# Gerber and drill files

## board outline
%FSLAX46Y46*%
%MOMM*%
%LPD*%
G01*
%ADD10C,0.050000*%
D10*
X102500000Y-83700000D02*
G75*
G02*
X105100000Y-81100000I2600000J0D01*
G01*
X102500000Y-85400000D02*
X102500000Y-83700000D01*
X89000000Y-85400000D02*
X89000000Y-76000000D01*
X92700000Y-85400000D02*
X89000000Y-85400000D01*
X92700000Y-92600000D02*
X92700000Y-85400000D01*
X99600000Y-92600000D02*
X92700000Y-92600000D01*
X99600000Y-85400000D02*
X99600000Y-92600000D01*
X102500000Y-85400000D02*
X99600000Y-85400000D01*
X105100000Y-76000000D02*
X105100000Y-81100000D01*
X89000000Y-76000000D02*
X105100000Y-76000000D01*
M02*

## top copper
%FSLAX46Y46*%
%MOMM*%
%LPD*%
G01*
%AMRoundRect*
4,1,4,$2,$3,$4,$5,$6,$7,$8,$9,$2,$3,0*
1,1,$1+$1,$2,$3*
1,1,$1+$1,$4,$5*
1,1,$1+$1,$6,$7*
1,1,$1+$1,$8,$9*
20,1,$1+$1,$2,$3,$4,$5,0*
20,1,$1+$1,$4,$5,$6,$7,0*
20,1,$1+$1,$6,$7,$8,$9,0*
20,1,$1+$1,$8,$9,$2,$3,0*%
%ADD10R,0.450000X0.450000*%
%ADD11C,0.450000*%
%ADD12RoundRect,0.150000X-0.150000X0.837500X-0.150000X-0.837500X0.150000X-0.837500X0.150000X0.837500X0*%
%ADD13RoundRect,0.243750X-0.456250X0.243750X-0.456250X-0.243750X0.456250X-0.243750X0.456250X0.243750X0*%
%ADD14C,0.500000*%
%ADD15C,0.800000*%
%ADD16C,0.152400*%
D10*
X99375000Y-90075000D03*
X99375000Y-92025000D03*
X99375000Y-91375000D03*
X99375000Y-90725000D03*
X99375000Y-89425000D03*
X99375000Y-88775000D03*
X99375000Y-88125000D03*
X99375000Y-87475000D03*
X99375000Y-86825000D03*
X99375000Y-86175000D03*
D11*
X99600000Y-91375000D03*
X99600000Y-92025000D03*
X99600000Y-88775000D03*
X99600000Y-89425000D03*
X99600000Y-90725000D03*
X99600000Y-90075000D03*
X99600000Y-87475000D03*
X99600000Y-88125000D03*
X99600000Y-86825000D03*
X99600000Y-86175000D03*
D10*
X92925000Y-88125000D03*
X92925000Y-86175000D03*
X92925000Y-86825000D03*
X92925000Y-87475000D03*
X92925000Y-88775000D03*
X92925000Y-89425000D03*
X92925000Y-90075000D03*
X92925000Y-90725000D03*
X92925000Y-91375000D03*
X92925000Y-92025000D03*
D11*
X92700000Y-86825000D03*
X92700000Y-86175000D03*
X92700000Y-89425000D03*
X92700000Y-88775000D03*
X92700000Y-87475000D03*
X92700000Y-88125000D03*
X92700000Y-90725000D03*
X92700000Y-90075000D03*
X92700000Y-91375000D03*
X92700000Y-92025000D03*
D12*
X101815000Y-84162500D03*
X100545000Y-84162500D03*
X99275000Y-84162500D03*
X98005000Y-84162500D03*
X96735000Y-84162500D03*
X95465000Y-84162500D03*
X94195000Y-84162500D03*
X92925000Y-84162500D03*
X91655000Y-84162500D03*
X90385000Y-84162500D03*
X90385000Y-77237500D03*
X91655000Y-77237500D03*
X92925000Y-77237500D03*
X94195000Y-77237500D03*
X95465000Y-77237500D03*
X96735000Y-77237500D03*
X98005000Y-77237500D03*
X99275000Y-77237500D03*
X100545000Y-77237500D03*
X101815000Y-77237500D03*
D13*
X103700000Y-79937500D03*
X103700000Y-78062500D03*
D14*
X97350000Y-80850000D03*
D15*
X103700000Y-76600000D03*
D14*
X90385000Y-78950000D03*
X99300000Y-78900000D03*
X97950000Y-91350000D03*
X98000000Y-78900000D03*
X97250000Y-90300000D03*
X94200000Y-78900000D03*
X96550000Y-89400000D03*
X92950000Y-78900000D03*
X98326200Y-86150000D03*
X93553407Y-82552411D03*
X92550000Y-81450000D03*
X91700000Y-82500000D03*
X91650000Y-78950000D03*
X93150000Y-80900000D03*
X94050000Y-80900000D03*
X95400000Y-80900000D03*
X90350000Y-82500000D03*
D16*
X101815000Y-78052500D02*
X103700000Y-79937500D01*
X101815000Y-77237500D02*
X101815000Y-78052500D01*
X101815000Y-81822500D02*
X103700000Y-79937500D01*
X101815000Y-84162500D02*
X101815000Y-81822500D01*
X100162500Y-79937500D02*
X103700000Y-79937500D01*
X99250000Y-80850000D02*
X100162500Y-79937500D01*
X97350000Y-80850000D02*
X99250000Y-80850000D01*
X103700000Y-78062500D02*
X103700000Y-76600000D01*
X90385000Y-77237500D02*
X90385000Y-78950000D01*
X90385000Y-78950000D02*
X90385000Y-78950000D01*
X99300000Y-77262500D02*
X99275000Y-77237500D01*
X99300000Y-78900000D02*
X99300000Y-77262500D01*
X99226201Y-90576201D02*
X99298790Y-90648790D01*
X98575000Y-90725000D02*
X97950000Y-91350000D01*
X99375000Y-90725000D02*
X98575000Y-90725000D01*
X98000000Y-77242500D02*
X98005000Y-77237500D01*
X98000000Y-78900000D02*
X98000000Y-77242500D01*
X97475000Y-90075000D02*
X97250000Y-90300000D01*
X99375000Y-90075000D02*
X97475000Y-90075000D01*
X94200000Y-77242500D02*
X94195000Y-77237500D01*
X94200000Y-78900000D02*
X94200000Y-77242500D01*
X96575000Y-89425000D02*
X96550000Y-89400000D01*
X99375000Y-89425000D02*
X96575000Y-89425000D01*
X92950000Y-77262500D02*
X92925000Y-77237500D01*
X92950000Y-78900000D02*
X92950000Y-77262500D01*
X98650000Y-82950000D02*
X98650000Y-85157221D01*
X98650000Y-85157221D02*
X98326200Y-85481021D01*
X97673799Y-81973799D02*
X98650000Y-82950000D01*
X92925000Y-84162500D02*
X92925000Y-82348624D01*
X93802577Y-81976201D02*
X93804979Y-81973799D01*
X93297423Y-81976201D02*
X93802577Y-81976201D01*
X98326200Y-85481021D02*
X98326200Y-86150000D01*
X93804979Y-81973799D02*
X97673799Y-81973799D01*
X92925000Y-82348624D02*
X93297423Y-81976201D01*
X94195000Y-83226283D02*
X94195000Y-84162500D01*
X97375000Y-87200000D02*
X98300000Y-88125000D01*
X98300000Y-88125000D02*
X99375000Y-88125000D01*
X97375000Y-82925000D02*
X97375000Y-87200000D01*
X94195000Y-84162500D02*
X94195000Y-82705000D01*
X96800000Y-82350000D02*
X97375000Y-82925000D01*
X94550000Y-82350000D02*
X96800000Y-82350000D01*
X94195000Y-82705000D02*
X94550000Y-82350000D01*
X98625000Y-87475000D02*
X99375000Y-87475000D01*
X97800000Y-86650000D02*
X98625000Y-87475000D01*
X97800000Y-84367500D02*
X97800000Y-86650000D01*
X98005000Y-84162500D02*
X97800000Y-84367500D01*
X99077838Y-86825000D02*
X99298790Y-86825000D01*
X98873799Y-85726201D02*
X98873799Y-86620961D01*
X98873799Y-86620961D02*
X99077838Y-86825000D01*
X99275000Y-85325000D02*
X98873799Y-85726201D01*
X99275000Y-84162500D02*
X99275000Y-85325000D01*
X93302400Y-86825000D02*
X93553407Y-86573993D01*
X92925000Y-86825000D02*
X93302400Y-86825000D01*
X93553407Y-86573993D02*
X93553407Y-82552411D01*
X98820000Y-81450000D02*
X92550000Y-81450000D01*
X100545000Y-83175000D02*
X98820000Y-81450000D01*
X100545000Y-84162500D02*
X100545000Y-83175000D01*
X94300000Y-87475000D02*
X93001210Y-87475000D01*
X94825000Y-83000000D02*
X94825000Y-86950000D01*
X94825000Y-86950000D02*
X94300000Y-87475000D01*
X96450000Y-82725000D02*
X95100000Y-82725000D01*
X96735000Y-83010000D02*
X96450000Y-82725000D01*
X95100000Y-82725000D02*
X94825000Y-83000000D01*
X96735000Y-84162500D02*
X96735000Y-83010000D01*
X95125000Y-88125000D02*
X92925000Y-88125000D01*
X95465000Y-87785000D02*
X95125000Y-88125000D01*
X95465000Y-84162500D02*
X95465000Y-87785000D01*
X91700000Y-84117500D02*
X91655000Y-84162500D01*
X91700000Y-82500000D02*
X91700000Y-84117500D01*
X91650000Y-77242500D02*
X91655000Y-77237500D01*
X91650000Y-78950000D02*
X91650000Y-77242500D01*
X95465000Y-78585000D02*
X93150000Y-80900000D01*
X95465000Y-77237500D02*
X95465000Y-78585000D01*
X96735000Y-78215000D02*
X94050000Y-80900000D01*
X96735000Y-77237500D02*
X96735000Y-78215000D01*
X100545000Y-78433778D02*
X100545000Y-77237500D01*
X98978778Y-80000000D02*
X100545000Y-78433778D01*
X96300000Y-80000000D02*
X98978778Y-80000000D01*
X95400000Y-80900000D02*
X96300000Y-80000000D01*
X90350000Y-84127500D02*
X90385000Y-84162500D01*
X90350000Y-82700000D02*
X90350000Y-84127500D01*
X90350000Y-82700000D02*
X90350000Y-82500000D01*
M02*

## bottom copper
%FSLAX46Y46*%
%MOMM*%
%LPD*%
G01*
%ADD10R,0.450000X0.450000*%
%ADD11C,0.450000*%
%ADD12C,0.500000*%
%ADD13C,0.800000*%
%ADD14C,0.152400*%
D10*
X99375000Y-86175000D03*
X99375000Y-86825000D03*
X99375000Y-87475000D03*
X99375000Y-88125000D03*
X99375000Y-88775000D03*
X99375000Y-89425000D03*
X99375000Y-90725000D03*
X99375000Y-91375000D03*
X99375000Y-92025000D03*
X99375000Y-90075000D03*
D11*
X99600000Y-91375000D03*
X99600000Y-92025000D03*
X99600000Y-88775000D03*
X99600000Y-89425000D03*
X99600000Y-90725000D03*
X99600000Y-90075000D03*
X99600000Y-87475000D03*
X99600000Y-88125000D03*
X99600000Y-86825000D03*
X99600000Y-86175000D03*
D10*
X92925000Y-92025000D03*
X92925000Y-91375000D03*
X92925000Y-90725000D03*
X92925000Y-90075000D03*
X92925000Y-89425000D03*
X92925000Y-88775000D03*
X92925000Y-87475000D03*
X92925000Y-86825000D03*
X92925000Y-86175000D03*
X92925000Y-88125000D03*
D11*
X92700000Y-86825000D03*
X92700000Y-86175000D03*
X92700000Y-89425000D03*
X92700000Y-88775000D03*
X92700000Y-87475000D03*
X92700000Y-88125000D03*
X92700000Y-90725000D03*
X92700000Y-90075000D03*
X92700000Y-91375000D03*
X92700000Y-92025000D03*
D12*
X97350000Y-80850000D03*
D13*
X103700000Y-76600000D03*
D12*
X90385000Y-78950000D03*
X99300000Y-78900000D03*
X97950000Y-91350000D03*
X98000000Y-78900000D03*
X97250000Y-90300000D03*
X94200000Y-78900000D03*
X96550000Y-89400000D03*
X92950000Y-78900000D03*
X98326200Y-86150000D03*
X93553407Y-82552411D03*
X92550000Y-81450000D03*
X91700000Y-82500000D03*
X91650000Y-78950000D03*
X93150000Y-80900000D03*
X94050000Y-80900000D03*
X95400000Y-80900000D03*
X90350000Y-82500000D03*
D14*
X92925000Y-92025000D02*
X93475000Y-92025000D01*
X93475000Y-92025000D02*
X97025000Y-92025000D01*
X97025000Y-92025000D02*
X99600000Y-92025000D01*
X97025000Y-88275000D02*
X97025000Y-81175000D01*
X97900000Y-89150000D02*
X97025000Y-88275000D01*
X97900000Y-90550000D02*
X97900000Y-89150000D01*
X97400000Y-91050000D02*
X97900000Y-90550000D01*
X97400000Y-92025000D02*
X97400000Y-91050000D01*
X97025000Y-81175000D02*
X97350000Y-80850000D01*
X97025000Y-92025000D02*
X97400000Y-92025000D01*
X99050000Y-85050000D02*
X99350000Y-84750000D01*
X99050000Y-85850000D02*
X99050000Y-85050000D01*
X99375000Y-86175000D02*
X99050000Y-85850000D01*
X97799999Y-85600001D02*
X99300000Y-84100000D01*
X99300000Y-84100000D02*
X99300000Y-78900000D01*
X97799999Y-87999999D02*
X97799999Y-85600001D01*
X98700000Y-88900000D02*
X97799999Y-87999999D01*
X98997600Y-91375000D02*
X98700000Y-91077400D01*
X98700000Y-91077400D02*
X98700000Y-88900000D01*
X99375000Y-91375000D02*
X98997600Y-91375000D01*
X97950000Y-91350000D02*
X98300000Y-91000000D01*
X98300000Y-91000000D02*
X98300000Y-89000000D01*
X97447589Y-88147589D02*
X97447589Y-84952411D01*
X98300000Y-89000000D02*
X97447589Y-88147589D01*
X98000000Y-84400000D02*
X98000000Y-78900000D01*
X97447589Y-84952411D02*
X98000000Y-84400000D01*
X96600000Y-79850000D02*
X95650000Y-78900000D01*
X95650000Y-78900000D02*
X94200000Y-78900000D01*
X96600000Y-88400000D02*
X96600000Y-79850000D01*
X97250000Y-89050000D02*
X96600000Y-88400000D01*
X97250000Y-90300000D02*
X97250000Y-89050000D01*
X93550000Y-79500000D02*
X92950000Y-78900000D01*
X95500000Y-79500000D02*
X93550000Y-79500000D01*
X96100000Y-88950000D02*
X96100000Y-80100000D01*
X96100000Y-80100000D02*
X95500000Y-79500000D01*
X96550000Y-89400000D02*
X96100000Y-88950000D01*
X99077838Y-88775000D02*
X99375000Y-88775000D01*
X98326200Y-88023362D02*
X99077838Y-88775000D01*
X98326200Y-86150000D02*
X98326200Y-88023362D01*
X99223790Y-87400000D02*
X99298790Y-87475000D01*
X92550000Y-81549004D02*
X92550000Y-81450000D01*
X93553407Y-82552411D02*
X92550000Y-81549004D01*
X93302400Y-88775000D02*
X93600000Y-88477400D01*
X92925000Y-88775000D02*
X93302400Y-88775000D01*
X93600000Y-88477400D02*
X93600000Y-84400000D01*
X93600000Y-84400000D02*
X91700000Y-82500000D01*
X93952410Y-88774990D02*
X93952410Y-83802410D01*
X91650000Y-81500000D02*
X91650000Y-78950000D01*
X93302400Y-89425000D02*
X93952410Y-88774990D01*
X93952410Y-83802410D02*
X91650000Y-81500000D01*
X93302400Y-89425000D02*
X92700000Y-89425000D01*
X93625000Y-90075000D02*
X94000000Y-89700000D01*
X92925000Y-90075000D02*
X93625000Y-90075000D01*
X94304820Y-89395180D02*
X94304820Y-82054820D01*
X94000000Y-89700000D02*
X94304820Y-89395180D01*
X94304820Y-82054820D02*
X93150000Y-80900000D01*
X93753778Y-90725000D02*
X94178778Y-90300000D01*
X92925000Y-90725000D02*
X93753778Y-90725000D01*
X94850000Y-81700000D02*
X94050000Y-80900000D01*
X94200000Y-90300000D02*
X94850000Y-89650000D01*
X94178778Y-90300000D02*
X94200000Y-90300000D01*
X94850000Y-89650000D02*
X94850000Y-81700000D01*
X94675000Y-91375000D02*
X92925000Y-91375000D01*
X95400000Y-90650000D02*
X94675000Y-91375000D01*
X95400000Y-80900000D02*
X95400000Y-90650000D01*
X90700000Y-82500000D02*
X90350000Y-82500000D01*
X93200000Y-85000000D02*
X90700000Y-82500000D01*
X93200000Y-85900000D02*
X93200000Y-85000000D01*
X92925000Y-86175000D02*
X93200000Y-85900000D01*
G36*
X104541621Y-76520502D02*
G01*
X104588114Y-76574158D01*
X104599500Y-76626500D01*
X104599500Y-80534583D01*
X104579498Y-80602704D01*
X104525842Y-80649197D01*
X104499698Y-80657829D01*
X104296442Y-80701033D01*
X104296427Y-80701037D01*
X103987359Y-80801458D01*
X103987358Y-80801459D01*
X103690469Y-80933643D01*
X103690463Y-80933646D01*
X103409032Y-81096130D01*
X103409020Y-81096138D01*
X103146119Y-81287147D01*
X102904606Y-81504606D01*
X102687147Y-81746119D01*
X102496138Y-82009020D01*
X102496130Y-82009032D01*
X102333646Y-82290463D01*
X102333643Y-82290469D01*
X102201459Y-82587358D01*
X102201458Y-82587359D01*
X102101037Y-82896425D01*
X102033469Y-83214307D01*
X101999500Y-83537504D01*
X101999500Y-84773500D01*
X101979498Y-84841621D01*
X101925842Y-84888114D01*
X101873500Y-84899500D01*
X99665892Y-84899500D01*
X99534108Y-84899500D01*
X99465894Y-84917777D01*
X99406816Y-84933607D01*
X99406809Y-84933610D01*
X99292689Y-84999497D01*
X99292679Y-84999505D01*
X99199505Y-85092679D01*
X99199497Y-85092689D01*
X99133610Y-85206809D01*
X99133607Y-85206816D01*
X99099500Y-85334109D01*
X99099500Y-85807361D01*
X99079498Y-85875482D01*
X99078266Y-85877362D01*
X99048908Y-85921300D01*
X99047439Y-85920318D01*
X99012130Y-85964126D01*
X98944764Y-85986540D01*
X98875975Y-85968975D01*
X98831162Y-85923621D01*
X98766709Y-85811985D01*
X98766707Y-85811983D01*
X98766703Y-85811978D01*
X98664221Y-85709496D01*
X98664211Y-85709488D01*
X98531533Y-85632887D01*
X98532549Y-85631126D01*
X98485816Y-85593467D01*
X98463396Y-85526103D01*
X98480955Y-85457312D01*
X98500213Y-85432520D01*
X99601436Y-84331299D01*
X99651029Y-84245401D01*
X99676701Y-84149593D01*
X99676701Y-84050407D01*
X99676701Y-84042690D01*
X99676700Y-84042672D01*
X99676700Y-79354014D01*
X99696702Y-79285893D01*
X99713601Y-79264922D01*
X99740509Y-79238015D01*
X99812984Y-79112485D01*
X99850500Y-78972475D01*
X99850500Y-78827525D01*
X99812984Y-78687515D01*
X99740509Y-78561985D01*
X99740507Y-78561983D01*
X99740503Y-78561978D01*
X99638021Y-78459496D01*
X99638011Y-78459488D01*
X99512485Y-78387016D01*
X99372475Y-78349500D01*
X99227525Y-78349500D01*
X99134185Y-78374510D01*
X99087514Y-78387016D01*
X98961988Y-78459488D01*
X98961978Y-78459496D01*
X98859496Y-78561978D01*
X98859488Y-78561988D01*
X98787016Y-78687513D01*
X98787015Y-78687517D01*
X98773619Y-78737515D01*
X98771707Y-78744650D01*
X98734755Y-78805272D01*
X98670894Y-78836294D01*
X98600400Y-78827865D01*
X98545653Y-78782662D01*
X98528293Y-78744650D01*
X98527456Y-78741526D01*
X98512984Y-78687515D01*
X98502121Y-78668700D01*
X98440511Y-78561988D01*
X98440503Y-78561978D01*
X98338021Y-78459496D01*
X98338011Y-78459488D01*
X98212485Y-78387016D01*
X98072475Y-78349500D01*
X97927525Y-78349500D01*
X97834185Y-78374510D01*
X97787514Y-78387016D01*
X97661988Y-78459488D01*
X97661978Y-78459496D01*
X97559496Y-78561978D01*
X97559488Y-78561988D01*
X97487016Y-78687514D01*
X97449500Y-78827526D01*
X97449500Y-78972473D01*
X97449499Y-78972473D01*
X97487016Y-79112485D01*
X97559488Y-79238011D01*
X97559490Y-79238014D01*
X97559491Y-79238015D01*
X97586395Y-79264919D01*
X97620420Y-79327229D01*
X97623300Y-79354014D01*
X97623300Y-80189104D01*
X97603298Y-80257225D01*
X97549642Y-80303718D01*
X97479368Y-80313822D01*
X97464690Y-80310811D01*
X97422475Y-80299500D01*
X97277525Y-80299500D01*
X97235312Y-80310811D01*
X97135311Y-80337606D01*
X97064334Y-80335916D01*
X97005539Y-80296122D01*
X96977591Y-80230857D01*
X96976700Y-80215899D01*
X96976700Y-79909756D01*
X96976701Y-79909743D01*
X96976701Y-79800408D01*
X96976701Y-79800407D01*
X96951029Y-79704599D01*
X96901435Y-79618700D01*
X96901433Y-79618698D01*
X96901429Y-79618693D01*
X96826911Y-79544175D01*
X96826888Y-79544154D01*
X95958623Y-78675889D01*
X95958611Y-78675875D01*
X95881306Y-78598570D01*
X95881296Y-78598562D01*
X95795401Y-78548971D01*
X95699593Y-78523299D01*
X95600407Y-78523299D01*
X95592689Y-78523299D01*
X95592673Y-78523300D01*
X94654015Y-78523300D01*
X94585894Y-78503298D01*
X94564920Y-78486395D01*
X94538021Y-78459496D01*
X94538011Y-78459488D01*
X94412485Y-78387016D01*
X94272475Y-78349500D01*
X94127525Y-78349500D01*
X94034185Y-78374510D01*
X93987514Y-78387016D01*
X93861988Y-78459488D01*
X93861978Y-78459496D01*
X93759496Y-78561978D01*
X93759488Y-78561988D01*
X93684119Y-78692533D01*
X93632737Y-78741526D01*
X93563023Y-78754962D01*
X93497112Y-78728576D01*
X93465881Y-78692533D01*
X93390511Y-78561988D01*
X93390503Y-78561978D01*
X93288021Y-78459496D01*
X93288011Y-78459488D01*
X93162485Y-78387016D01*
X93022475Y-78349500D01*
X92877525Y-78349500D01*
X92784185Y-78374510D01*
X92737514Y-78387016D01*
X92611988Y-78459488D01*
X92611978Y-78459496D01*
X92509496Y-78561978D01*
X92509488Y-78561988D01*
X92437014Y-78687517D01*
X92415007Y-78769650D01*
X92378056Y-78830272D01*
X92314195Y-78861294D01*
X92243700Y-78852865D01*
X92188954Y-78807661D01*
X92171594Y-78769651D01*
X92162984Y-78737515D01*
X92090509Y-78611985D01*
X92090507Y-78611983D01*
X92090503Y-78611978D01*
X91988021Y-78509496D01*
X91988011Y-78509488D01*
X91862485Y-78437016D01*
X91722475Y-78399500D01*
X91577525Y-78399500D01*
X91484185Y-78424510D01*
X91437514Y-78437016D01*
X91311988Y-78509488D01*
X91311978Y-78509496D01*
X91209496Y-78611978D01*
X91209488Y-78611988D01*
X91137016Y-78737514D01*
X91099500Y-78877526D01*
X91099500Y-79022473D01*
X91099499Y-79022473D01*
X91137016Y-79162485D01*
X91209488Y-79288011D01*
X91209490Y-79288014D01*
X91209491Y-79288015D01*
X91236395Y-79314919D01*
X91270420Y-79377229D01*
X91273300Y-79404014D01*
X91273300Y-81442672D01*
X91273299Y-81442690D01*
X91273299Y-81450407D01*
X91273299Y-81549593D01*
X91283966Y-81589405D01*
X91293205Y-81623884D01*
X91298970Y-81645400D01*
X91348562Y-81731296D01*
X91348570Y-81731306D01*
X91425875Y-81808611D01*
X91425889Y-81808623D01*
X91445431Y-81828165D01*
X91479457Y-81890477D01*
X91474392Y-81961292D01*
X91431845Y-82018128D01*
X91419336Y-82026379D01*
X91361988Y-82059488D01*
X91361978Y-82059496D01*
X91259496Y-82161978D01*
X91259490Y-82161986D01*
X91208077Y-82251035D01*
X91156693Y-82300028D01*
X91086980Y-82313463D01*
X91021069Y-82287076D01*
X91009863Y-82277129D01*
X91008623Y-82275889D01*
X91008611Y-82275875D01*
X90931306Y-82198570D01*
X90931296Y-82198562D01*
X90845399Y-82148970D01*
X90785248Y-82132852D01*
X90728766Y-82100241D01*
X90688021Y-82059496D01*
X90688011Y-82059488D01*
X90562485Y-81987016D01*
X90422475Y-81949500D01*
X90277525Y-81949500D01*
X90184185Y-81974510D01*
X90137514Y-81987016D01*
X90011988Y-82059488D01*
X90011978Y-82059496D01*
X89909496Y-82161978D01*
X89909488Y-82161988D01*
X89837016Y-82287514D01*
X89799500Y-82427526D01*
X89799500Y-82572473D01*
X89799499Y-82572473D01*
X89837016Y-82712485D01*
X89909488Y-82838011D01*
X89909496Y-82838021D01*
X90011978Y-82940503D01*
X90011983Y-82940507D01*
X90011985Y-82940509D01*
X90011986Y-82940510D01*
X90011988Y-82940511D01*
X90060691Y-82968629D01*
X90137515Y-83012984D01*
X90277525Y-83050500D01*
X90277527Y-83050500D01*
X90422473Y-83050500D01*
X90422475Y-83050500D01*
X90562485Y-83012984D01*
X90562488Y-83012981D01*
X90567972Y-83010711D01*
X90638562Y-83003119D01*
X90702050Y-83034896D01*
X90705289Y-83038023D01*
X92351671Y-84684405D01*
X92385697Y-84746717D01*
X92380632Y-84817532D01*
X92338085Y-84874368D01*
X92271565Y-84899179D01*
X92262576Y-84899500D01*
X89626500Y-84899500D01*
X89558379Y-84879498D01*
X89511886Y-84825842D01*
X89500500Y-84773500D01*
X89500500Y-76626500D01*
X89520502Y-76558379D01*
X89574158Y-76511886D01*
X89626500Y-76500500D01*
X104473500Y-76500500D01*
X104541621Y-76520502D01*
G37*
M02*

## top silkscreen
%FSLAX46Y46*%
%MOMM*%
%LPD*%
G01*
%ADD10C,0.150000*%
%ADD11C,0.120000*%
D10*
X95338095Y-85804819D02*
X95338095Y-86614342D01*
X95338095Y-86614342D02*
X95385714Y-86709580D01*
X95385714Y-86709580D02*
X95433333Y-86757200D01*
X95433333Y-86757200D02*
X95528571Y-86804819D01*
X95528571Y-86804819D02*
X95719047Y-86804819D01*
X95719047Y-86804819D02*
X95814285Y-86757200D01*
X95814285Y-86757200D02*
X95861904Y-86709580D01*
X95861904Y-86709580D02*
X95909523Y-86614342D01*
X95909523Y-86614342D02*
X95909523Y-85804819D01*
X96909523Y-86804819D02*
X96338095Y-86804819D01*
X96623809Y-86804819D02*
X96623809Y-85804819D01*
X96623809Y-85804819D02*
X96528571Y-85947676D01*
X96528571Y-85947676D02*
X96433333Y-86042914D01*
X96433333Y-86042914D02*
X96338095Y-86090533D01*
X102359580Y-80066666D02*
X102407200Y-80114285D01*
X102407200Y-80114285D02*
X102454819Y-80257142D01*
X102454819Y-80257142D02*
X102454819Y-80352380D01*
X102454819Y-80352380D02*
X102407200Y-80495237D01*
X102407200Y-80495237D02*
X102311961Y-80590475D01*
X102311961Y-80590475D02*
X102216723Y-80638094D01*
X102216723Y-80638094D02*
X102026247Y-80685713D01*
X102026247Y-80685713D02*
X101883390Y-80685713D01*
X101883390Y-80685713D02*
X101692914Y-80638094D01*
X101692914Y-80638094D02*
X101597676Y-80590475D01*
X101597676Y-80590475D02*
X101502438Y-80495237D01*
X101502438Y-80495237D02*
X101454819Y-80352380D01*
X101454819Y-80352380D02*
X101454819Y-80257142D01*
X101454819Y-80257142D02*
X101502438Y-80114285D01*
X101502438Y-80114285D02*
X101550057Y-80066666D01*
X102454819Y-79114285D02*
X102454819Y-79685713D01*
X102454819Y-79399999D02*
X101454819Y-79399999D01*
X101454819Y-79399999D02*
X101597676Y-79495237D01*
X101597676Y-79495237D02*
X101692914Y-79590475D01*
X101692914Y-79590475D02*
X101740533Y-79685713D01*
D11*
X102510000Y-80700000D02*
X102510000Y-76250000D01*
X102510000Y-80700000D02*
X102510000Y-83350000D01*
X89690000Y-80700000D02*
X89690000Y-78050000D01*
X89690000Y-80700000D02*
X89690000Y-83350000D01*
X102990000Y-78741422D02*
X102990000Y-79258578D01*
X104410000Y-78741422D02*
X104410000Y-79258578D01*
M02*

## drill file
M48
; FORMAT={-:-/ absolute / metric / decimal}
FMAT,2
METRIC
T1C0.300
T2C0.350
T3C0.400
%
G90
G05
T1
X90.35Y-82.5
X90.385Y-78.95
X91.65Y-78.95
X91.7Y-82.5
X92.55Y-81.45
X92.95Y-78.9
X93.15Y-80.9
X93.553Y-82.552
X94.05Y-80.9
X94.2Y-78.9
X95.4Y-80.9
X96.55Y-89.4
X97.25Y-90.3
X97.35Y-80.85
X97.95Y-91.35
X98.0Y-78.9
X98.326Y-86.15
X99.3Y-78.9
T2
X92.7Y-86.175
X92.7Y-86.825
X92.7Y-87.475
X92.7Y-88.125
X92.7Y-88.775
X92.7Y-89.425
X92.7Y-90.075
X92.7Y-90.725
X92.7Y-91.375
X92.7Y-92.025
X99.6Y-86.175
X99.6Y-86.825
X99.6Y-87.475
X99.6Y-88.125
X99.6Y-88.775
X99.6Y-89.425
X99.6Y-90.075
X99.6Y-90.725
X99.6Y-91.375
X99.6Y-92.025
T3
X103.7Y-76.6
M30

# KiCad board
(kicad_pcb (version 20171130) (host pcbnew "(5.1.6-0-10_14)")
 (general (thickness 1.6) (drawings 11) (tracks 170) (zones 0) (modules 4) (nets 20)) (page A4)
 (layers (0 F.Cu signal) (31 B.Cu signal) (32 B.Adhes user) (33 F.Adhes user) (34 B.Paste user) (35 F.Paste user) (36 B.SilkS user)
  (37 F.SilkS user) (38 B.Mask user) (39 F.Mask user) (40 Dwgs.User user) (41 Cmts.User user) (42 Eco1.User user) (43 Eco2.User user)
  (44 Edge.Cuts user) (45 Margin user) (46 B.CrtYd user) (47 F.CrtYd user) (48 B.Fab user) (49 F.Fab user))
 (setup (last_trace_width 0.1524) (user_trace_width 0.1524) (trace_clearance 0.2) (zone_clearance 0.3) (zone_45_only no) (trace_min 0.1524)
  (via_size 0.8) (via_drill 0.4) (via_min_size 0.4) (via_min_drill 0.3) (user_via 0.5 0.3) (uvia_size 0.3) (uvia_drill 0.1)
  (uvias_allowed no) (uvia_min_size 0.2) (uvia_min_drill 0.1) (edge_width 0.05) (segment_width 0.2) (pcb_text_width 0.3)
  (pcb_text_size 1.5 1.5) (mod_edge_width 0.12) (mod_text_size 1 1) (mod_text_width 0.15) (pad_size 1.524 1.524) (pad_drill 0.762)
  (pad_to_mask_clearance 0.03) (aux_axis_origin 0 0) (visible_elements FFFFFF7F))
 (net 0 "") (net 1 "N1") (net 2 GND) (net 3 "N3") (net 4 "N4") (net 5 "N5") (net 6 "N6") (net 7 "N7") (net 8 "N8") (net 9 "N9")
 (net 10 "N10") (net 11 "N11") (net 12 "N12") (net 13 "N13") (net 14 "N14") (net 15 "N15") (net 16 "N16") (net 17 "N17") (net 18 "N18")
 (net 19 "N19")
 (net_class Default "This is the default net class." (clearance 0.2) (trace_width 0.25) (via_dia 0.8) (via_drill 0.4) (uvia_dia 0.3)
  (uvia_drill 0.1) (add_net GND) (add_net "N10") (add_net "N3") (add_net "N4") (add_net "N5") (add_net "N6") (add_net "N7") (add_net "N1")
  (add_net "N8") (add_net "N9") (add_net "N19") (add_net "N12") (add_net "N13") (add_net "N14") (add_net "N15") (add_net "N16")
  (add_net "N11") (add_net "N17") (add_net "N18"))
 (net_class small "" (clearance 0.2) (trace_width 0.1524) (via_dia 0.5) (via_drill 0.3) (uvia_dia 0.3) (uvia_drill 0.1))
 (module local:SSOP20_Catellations (layer F.Cu) (at 99.6 89.1)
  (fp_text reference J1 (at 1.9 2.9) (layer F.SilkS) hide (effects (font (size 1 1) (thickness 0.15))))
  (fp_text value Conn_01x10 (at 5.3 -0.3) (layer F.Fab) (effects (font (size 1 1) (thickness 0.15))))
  (pad 7 smd rect (at -0.225 0.975) (size 0.45 0.45) (layers F.Cu F.Paste F.Mask) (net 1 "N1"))
  (pad 1 smd rect (at -0.225 -2.925) (size 0.45 0.45) (layers B.Cu B.Paste B.Mask) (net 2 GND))
  (pad 2 smd rect (at -0.225 -2.275) (size 0.45 0.45) (layers B.Cu B.Paste B.Mask) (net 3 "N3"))
  (pad 3 smd rect (at -0.225 -1.625) (size 0.45 0.45) (layers B.Cu B.Paste B.Mask) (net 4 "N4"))
  (pad 4 smd rect (at -0.225 -0.975) (size 0.45 0.45) (layers B.Cu B.Paste B.Mask) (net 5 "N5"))
  (pad 5 smd rect (at -0.225 -0.325) (size 0.45 0.45) (layers B.Cu B.Paste B.Mask) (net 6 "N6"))
  (pad 6 smd rect (at -0.225 0.325) (size 0.45 0.45) (layers B.Cu B.Paste B.Mask) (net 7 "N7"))
  (pad 8 smd rect (at -0.225 1.625) (size 0.45 0.45) (layers B.Cu B.Paste B.Mask) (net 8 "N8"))
  (pad 9 smd rect (at -0.225 2.275) (size 0.45 0.45) (layers B.Cu B.Paste B.Mask) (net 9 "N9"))
  (pad 10 smd rect (at -0.225 2.925) (size 0.45 0.45) (layers B.Cu B.Paste B.Mask) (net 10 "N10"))
  (pad 10 smd rect (at -0.225 2.925) (size 0.45 0.45) (layers F.Cu F.Paste F.Mask) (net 10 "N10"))
  (pad 9 smd rect (at -0.225 2.275) (size 0.45 0.45) (layers F.Cu F.Paste F.Mask) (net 9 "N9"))
  (pad 8 smd rect (at -0.225 1.625) (size 0.45 0.45) (layers F.Cu F.Paste F.Mask) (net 8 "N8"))
  (pad 7 smd rect (at -0.225 0.975) (size 0.45 0.45) (layers B.Cu B.Paste B.Mask) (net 1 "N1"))
  (pad 6 smd rect (at -0.225 0.325) (size 0.45 0.45) (layers F.Cu F.Paste F.Mask) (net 7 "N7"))
  (pad 5 smd rect (at -0.225 -0.325) (size 0.45 0.45) (layers F.Cu F.Paste F.Mask) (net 6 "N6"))
  (pad 4 smd rect (at -0.225 -0.975) (size 0.45 0.45) (layers F.Cu F.Paste F.Mask) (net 5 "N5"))
  (pad 3 smd rect (at -0.225 -1.625) (size 0.45 0.45) (layers F.Cu F.Paste F.Mask) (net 4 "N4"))
  (pad 2 smd rect (at -0.225 -2.275) (size 0.45 0.45) (layers F.Cu F.Paste F.Mask) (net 3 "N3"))
  (pad 1 smd rect (at -0.225 -2.925) (size 0.45 0.45) (layers F.Cu F.Paste F.Mask) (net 2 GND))
  (pad 9 thru_hole circle (at 0 2.275) (size 0.45 0.45) (drill 0.35) (layers *.Cu *.Mask) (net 9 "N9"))
  (pad 10 thru_hole circle (at 0 2.925) (size 0.45 0.45) (drill 0.35) (layers *.Cu *.Mask) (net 10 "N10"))
  (pad 5 thru_hole circle (at 0 -0.325) (size 0.45 0.45) (drill 0.35) (layers *.Cu *.Mask) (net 6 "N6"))
  (pad 6 thru_hole circle (at 0 0.325) (size 0.45 0.45) (drill 0.35) (layers *.Cu *.Mask) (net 7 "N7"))
  (pad 8 thru_hole circle (at 0 1.625) (size 0.45 0.45) (drill 0.35) (layers *.Cu *.Mask) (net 8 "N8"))
  (pad 7 thru_hole circle (at 0 0.975) (size 0.45 0.45) (drill 0.35) (layers *.Cu *.Mask) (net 1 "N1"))
  (pad 3 thru_hole circle (at 0 -1.625) (size 0.45 0.45) (drill 0.35) (layers *.Cu *.Mask) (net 4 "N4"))
  (pad 4 thru_hole circle (at 0 -0.975) (size 0.45 0.45) (drill 0.35) (layers *.Cu *.Mask) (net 5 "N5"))
  (pad 2 thru_hole circle (at 0 -2.275) (size 0.45 0.45) (drill 0.35) (layers *.Cu *.Mask) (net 3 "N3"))
  (pad 1 thru_hole circle (at 0 -2.925) (size 0.45 0.45) (drill 0.35) (layers *.Cu *.Mask) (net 2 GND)))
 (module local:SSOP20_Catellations (layer F.Cu) (at 92.7 89.1 180)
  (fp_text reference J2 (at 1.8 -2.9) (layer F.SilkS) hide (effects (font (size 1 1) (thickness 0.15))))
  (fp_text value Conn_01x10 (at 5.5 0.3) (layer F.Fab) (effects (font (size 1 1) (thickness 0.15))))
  (pad 7 smd rect (at -0.225 0.975 180) (size 0.45 0.45) (layers F.Cu F.Paste F.Mask) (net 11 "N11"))
  (pad 1 smd rect (at -0.225 -2.925 180) (size 0.45 0.45) (layers B.Cu B.Paste B.Mask) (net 10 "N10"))
  (pad 2 smd rect (at -0.225 -2.275 180) (size 0.45 0.45) (layers B.Cu B.Paste B.Mask) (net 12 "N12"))
  (pad 3 smd rect (at -0.225 -1.625 180) (size 0.45 0.45) (layers B.Cu B.Paste B.Mask) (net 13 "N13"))
  (pad 4 smd rect (at -0.225 -0.975 180) (size 0.45 0.45) (layers B.Cu B.Paste B.Mask) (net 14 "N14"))
  (pad 5 smd rect (at -0.225 -0.325 180) (size 0.45 0.45) (layers B.Cu B.Paste B.Mask) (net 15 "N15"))
  (pad 6 smd rect (at -0.225 0.325 180) (size 0.45 0.45) (layers B.Cu B.Paste B.Mask) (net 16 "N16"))
  (pad 8 smd rect (at -0.225 1.625 180) (size 0.45 0.45) (layers B.Cu B.Paste B.Mask) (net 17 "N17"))
  (pad 9 smd rect (at -0.225 2.275 180) (size 0.45 0.45) (layers B.Cu B.Paste B.Mask) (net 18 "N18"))
  (pad 10 smd rect (at -0.225 2.925 180) (size 0.45 0.45) (layers B.Cu B.Paste B.Mask) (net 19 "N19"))
  (pad 10 smd rect (at -0.225 2.925 180) (size 0.45 0.45) (layers F.Cu F.Paste F.Mask) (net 19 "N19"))
  (pad 9 smd rect (at -0.225 2.275 180) (size 0.45 0.45) (layers F.Cu F.Paste F.Mask) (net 18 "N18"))
  (pad 8 smd rect (at -0.225 1.625 180) (size 0.45 0.45) (layers F.Cu F.Paste F.Mask) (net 17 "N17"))
  (pad 7 smd rect (at -0.225 0.975 180) (size 0.45 0.45) (layers B.Cu B.Paste B.Mask) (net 11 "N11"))
  (pad 6 smd rect (at -0.225 0.325 180) (size 0.45 0.45) (layers F.Cu F.Paste F.Mask) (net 16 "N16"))
  (pad 5 smd rect (at -0.225 -0.325 180) (size 0.45 0.45) (layers F.Cu F.Paste F.Mask) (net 15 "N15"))
  (pad 4 smd rect (at -0.225 -0.975 180) (size 0.45 0.45) (layers F.Cu F.Paste F.Mask) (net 14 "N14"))
  (pad 3 smd rect (at -0.225 -1.625 180) (size 0.45 0.45) (layers F.Cu F.Paste F.Mask) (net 13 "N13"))
  (pad 2 smd rect (at -0.225 -2.275 180) (size 0.45 0.45) (layers F.Cu F.Paste F.Mask) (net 12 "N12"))
  (pad 1 smd rect (at -0.225 -2.925 180) (size 0.45 0.45) (layers F.Cu F.Paste F.Mask) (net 10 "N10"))
  (pad 9 thru_hole circle (at 0 2.275 180) (size 0.45 0.45) (drill 0.35) (layers *.Cu *.Mask) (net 18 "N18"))
  (pad 10 thru_hole circle (at 0 2.925 180) (size 0.45 0.45) (drill 0.35) (layers *.Cu *.Mask) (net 19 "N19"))
  (pad 5 thru_hole circle (at 0 -0.325 180) (size 0.45 0.45) (drill 0.35) (layers *.Cu *.Mask) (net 15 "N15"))
  (pad 6 thru_hole circle (at 0 0.325 180) (size 0.45 0.45) (drill 0.35) (layers *.Cu *.Mask) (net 16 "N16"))
  (pad 8 thru_hole circle (at 0 1.625 180) (size 0.45 0.45) (drill 0.35) (layers *.Cu *.Mask) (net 17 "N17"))
  (pad 7 thru_hole circle (at 0 0.975 180) (size 0.45 0.45) (drill 0.35) (layers *.Cu *.Mask) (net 11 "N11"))
  (pad 3 thru_hole circle (at 0 -1.625 180) (size 0.45 0.45) (drill 0.35) (layers *.Cu *.Mask) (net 13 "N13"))
  (pad 4 thru_hole circle (at 0 -0.975 180) (size 0.45 0.45) (drill 0.35) (layers *.Cu *.Mask) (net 14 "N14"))
  (pad 2 thru_hole circle (at 0 -2.275 180) (size 0.45 0.45) (drill 0.35) (layers *.Cu *.Mask) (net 12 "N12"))
  (pad 1 thru_hole circle (at 0 -2.925 180) (size 0.45 0.45) (drill 0.35) (layers *.Cu *.Mask) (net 10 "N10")))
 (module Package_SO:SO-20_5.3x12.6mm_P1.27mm (layer F.Cu) (at 96.1 80.7 270)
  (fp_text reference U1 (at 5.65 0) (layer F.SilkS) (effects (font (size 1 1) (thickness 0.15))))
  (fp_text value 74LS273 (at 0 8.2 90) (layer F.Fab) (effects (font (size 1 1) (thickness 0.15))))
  (fp_line (start 0 -6.41) (end -4.45 -6.41) (layer F.SilkS) (width 0.12))
  (fp_line (start 0 -6.41) (end 2.65 -6.41) (layer F.SilkS) (width 0.12))
  (fp_line (start 0 6.41) (end -2.65 6.41) (layer F.SilkS) (width 0.12))
  (fp_line (start 0 6.41) (end 2.65 6.41) (layer F.SilkS) (width 0.12))
  (pad 20 smd roundrect (at 3.4625 -5.715 270) (size 1.975 0.6) (layers F.Cu F.Paste F.Mask) (roundrect_rratio 0.25) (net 10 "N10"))
  (pad 19 smd roundrect (at 3.4625 -4.445 270) (size 1.975 0.6) (layers F.Cu F.Paste F.Mask) (roundrect_rratio 0.25) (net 18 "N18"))
  (pad 18 smd roundrect (at 3.4625 -3.175 270) (size 1.975 0.6) (layers F.Cu F.Paste F.Mask) (roundrect_rratio 0.25) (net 3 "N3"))
  (pad 17 smd roundrect (at 3.4625 -1.905 270) (size 1.975 0.6) (layers F.Cu F.Paste F.Mask) (roundrect_rratio 0.25) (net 4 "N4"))
  (pad 16 smd roundrect (at 3.4625 -0.635 270) (size 1.975 0.6) (layers F.Cu F.Paste F.Mask) (roundrect_rratio 0.25) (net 17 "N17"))
  (pad 15 smd roundrect (at 3.4625 0.635 270) (size 1.975 0.6) (layers F.Cu F.Paste F.Mask) (roundrect_rratio 0.25) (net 11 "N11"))
  (pad 14 smd roundrect (at 3.4625 1.905 270) (size 1.975 0.6) (layers F.Cu F.Paste F.Mask) (roundrect_rratio 0.25) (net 5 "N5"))
  (pad 13 smd roundrect (at 3.4625 3.175 270) (size 1.975 0.6) (layers F.Cu F.Paste F.Mask) (roundrect_rratio 0.25) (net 6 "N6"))
  (pad 12 smd roundrect (at 3.4625 4.445 270) (size 1.975 0.6) (layers F.Cu F.Paste F.Mask) (roundrect_rratio 0.25) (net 16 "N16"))
  (pad 11 smd roundrect (at 3.4625 5.715 270) (size 1.975 0.6) (layers F.Cu F.Paste F.Mask) (roundrect_rratio 0.25) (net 19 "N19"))
  (pad 10 smd roundrect (at -3.4625 5.715 270) (size 1.975 0.6) (layers F.Cu F.Paste F.Mask) (roundrect_rratio 0.25) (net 2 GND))
  (pad 9 smd roundrect (at -3.4625 4.445 270) (size 1.975 0.6) (layers F.Cu F.Paste F.Mask) (roundrect_rratio 0.25) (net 15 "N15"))
  (pad 8 smd roundrect (at -3.4625 3.175 270) (size 1.975 0.6) (layers F.Cu F.Paste F.Mask) (roundrect_rratio 0.25) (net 7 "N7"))
  (pad 7 smd roundrect (at -3.4625 1.905 270) (size 1.975 0.6) (layers F.Cu F.Paste F.Mask) (roundrect_rratio 0.25) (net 1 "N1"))
  (pad 6 smd roundrect (at -3.4625 0.635 270) (size 1.975 0.6) (layers F.Cu F.Paste F.Mask) (roundrect_rratio 0.25) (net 14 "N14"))
  (pad 5 smd roundrect (at -3.4625 -0.635 270) (size 1.975 0.6) (layers F.Cu F.Paste F.Mask) (roundrect_rratio 0.25) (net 13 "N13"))
  (pad 4 smd roundrect (at -3.4625 -1.905 270) (size 1.975 0.6) (layers F.Cu F.Paste F.Mask) (roundrect_rratio 0.25) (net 8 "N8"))
  (pad 3 smd roundrect (at -3.4625 -3.175 270) (size 1.975 0.6) (layers F.Cu F.Paste F.Mask) (roundrect_rratio 0.25) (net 9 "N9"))
  (pad 2 smd roundrect (at -3.4625 -4.445 270) (size 1.975 0.6) (layers F.Cu F.Paste F.Mask) (roundrect_rratio 0.25) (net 12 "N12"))
  (pad 1 smd roundrect (at -3.4625 -5.715 270) (size 1.975 0.6) (layers F.Cu F.Paste F.Mask) (roundrect_rratio 0.25) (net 10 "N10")))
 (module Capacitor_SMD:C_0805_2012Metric (layer F.Cu) (at 103.7 79 270)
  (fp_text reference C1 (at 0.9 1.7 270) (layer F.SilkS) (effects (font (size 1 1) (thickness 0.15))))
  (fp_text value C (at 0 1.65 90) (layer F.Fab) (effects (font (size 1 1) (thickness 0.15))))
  (fp_line (start -0.258578 0.71) (end 0.258578 0.71) (layer F.SilkS) (width 0.12))
  (fp_line (start -0.258578 -0.71) (end 0.258578 -0.71) (layer F.SilkS) (width 0.12))
  (pad 2 smd roundrect (at 0.9375 0 270) (size 0.975 1.4) (layers F.Cu F.Paste F.Mask) (roundrect_rratio 0.25) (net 10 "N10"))
  (pad 1 smd roundrect (at -0.9375 0 270) (size 0.975 1.4) (layers F.Cu F.Paste F.Mask) (roundrect_rratio 0.25) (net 2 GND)))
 (gr_arc (start 105.1 83.7) (end 105.1 81.1) (angle -90) (layer Edge.Cuts) (width 0.05))
 (gr_line (start 102.5 85.4) (end 102.5 83.7) (layer Edge.Cuts) (width 0.05))
 (gr_line (start 89 85.4) (end 89 76) (layer Edge.Cuts) (width 0.05))
 (gr_line (start 92.7 85.4) (end 89 85.4) (layer Edge.Cuts) (width 0.05))
 (gr_line (start 92.7 92.6) (end 92.7 85.4) (layer Edge.Cuts) (width 0.05))
 (gr_line (start 99.6 92.6) (end 92.7 92.6) (layer Edge.Cuts) (width 0.05))
 (gr_line (start 99.6 85.4) (end 99.6 92.6) (layer Edge.Cuts) (width 0.05))
 (gr_line (start 102.5 85.4) (end 99.6 85.4) (layer Edge.Cuts) (width 0.05))
 (gr_line (start 105.1 76) (end 105.1 81.1) (layer Edge.Cuts) (width 0.05))
 (gr_line (start 89 76) (end 105.1 76) (layer Edge.Cuts) (width 0.05))
 (segment (start 92.925 92.025) (end 93.475 92.025) (width 0.1524) (layer B.Cu) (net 10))
 (segment (start 93.475 92.025) (end 97.025 92.025) (width 0.1524) (layer B.Cu) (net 10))
 (via (at 97.35 80.85) (size 0.5) (drill 0.3) (layers F.Cu B.Cu) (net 10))
 (segment (start 97.025 92.025) (end 99.6 92.025) (width 0.1524) (layer B.Cu) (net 10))
 (segment (start 97.025 88.275) (end 97.025 81.175) (width 0.1524) (layer B.Cu) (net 10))
 (segment (start 97.9 89.15) (end 97.025 88.275) (width 0.1524) (layer B.Cu) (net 10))
 (segment (start 97.9 90.55) (end 97.9 89.15) (width 0.1524) (layer B.Cu) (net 10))
 (segment (start 97.4 91.05) (end 97.9 90.55) (width 0.1524) (layer B.Cu) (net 10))
 (segment (start 97.4 92.025) (end 97.4 91.05) (width 0.1524) (layer B.Cu) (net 10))
 (segment (start 97.025 81.175) (end 97.35 80.85) (width 0.1524) (layer B.Cu) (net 10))
 (segment (start 97.025 92.025) (end 97.4 92.025) (width 0.1524) (layer B.Cu) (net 10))
 (segment (start 101.815 78.0525) (end 103.7 79.9375) (width 0.1524) (layer F.Cu) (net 10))
 (segment (start 101.815 77.2375) (end 101.815 78.0525) (width 0.1524) (layer F.Cu) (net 10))
 (segment (start 101.815 81.8225) (end 103.7 79.9375) (width 0.1524) (layer F.Cu) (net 10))
 (segment (start 101.815 84.1625) (end 101.815 81.8225) (width 0.1524) (layer F.Cu) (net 10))
 (segment (start 100.1625 79.9375) (end 103.7 79.9375) (width 0.1524) (layer F.Cu) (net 10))
 (segment (start 99.25 80.85) (end 100.1625 79.9375) (width 0.1524) (layer F.Cu) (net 10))
 (segment (start 97.35 80.85) (end 99.25 80.85) (width 0.1524) (layer F.Cu) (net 10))
 (via (at 103.7 76.6) (size 0.8) (drill 0.4) (layers F.Cu B.Cu) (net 2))
 (segment (start 103.7 78.0625) (end 103.7 76.6) (width 0.1524) (layer F.Cu) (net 2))
 (segment (start 99.05 85.05) (end 99.35 84.75) (width 0.1524) (layer B.Cu) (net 2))
 (segment (start 99.05 85.85) (end 99.05 85.05) (width 0.1524) (layer B.Cu) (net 2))
 (segment (start 99.375 86.175) (end 99.05 85.85) (width 0.1524) (layer B.Cu) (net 2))
 (segment (start 90.385 77.2375) (end 90.385 78.95) (width 0.1524) (layer F.Cu) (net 2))
 (segment (start 90.385 78.95) (end 90.385 78.95) (width 0.1524) (layer F.Cu) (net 2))
 (via (at 90.385 78.95) (size 0.5) (drill 0.3) (layers F.Cu B.Cu) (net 2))
 (via (at 99.3 78.9) (size 0.5) (drill 0.3) (layers F.Cu B.Cu) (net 9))
 (segment (start 99.3 77.2625) (end 99.275 77.2375) (width 0.1524) (layer F.Cu) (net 9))
 (segment (start 99.3 78.9) (end 99.3 77.2625) (width 0.1524) (layer F.Cu) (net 9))
 (segment (start 97.799999 85.600001) (end 99.3 84.1) (width 0.1524) (layer B.Cu) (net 9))
 (segment (start 99.3 84.1) (end 99.3 78.9) (width 0.1524) (layer B.Cu) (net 9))
 (segment (start 97.799999 87.999999) (end 97.799999 85.600001) (width 0.1524) (layer B.Cu) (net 9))
 (segment (start 98.7 88.9) (end 97.799999 87.999999) (width 0.1524) (layer B.Cu) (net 9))
 (segment (start 98.9976 91.375) (end 98.7 91.0774) (width 0.1524) (layer B.Cu) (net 9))
 (segment (start 98.7 91.0774) (end 98.7 88.9) (width 0.1524) (layer B.Cu) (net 9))
 (segment (start 99.375 91.375) (end 98.9976 91.375) (width 0.1524) (layer B.Cu) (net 9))
 (segment (start 99.226201 90.576201) (end 99.29879 90.64879) (width 0.1524) (layer F.Cu) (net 8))
 (segment (start 98.575 90.725) (end 97.95 91.35) (width 0.1524) (layer F.Cu) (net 8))
 (via (at 97.95 91.35) (size 0.5) (drill 0.3) (layers F.Cu B.Cu) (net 8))
 (segment (start 99.375 90.725) (end 98.575 90.725) (width 0.1524) (layer F.Cu) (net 8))
 (segment (start 97.95 91.35) (end 98.3 91) (width 0.1524) (layer B.Cu) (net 8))
 (segment (start 98.3 91) (end 98.3 89) (width 0.1524) (layer B.Cu) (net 8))
 (segment (start 97.447589 88.147589) (end 97.447589 84.952411) (width 0.1524) (layer B.Cu) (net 8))
 (segment (start 98.3 89) (end 97.447589 88.147589) (width 0.1524) (layer B.Cu) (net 8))
 (via (at 98 78.9) (size 0.5) (drill 0.3) (layers F.Cu B.Cu) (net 8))
 (segment (start 98 84.4) (end 98 78.9) (width 0.1524) (layer B.Cu) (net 8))
 (segment (start 97.447589 84.952411) (end 98 84.4) (width 0.1524) (layer B.Cu) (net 8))
 (segment (start 98 77.2425) (end 98.005 77.2375) (width 0.1524) (layer F.Cu) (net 8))
 (segment (start 98 78.9) (end 98 77.2425) (width 0.1524) (layer F.Cu) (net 8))
 (via (at 97.25 90.3) (size 0.5) (drill 0.3) (layers F.Cu B.Cu) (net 1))
 (segment (start 97.475 90.075) (end 97.25 90.3) (width 0.1524) (layer F.Cu) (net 1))
 (segment (start 99.375 90.075) (end 97.475 90.075) (width 0.1524) (layer F.Cu) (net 1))
 (via (at 94.2 78.9) (size 0.5) (drill 0.3) (layers F.Cu B.Cu) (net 1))
 (segment (start 94.2 77.2425) (end 94.195 77.2375) (width 0.1524) (layer F.Cu) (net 1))
 (segment (start 94.2 78.9) (end 94.2 77.2425) (width 0.1524) (layer F.Cu) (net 1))
 (segment (start 96.6 79.85) (end 95.65 78.9) (width 0.1524) (layer B.Cu) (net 1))
 (segment (start 95.65 78.9) (end 94.2 78.9) (width 0.1524) (layer B.Cu) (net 1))
 (segment (start 96.6 88.4) (end 96.6 79.85) (width 0.1524) (layer B.Cu) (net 1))
 (segment (start 97.25 89.05) (end 96.6 88.4) (width 0.1524) (layer B.Cu) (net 1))
 (segment (start 97.25 90.3) (end 97.25 89.05) (width 0.1524) (layer B.Cu) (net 1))
 (via (at 96.55 89.4) (size 0.5) (drill 0.3) (layers F.Cu B.Cu) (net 7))
 (segment (start 96.575 89.425) (end 96.55 89.4) (width 0.1524) (layer F.Cu) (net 7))
 (segment (start 99.375 89.425) (end 96.575 89.425) (width 0.1524) (layer F.Cu) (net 7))
 (via (at 92.95 78.9) (size 0.5) (drill 0.3) (layers F.Cu B.Cu) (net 7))
 (segment (start 92.95 77.2625) (end 92.925 77.2375) (width 0.1524) (layer F.Cu) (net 7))
 (segment (start 92.95 78.9) (end 92.95 77.2625) (width 0.1524) (layer F.Cu) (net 7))
 (segment (start 93.55 79.5) (end 92.95 78.9) (width 0.1524) (layer B.Cu) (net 7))
 (segment (start 95.5 79.5) (end 93.55 79.5) (width 0.1524) (layer B.Cu) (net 7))
 (segment (start 96.1 88.95) (end 96.1 80.1) (width 0.1524) (layer B.Cu) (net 7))
 (segment (start 96.1 80.1) (end 95.5 79.5) (width 0.1524) (layer B.Cu) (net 7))
 (segment (start 96.55 89.4) (end 96.1 88.95) (width 0.1524) (layer B.Cu) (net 7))
 (via (at 98.3262 86.15) (size 0.5) (drill 0.3) (layers F.Cu B.Cu) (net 6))
 (segment (start 99.077838 88.775) (end 99.375 88.775) (width 0.1524) (layer B.Cu) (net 6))
 (segment (start 98.3262 88.023362) (end 99.077838 88.775) (width 0.1524) (layer B.Cu) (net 6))
 (segment (start 98.3262 86.15) (end 98.3262 88.023362) (width 0.1524) (layer B.Cu) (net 6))
 (segment (start 98.65 82.95) (end 98.65 85.157221) (width 0.1524) (layer F.Cu) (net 6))
 (segment (start 98.65 85.157221) (end 98.3262 85.481021) (width 0.1524) (layer F.Cu) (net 6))
 (segment (start 97.673799 81.973799) (end 98.65 82.95) (width 0.1524) (layer F.Cu) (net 6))
 (segment (start 92.925 84.1625) (end 92.925 82.348624) (width 0.1524) (layer F.Cu) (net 6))
 (segment (start 93.802577 81.976201) (end 93.804979 81.973799) (width 0.1524) (layer F.Cu) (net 6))
 (segment (start 93.297423 81.976201) (end 93.802577 81.976201) (width 0.1524) (layer F.Cu) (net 6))
 (segment (start 98.3262 85.481021) (end 98.3262 86.15) (width 0.1524) (layer F.Cu) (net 6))
 (segment (start 93.804979 81.973799) (end 97.673799 81.973799) (width 0.1524) (layer F.Cu) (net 6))
 (segment (start 92.925 82.348624) (end 93.297423 81.976201) (width 0.1524) (layer F.Cu) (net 6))
 (segment (start 94.195 83.226283) (end 94.195 84.1625) (width 0.1524) (layer F.Cu) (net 5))
 (segment (start 97.375 87.2) (end 98.3 88.125) (width 0.1524) (layer F.Cu) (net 5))
 (segment (start 98.3 88.125) (end 99.375 88.125) (width 0.1524) (layer F.Cu) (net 5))
 (segment (start 97.375 82.925) (end 97.375 87.2) (width 0.1524) (layer F.Cu) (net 5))
 (segment (start 94.195 84.1625) (end 94.195 82.705) (width 0.1524) (layer F.Cu) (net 5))
 (segment (start 96.8 82.35) (end 97.375 82.925) (width 0.1524) (layer F.Cu) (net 5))
 (segment (start 94.55 82.35) (end 96.8 82.35) (width 0.1524) (layer F.Cu) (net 5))
 (segment (start 94.195 82.705) (end 94.55 82.35) (width 0.1524) (layer F.Cu) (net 5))
 (segment (start 99.22379 87.4) (end 99.29879 87.475) (width 0.1524) (layer B.Cu) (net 4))
 (segment (start 98.625 87.475) (end 99.375 87.475) (width 0.1524) (layer F.Cu) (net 4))
 (segment (start 97.8 86.65) (end 98.625 87.475) (width 0.1524) (layer F.Cu) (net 4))
 (segment (start 97.8 84.3675) (end 97.8 86.65) (width 0.1524) (layer F.Cu) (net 4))
 (segment (start 98.005 84.1625) (end 97.8 84.3675) (width 0.1524) (layer F.Cu) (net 4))
 (segment (start 99.077838 86.825) (end 99.29879 86.825) (width 0.1524) (layer F.Cu) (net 3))
 (segment (start 98.873799 85.726201) (end 98.873799 86.620961) (width 0.1524) (layer F.Cu) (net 3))
 (segment (start 98.873799 86.620961) (end 99.077838 86.825) (width 0.1524) (layer F.Cu) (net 3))
 (segment (start 99.275 85.325) (end 98.873799 85.726201) (width 0.1524) (layer F.Cu) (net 3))
 (segment (start 99.275 84.1625) (end 99.275 85.325) (width 0.1524) (layer F.Cu) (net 3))
 (segment (start 93.3024 86.825) (end 93.553407 86.573993) (width 0.1524) (layer F.Cu) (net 18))
 (via (at 93.553407 82.552411) (size 0.5) (drill 0.3) (layers F.Cu B.Cu) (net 18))
 (segment (start 92.925 86.825) (end 93.3024 86.825) (width 0.1524) (layer F.Cu) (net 18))
 (segment (start 93.553407 86.573993) (end 93.553407 82.552411) (width 0.1524) (layer F.Cu) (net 18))
 (segment (start 98.82 81.45) (end 92.55 81.45) (width 0.1524) (layer F.Cu) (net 18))
 (segment (start 100.545 83.175) (end 98.82 81.45) (width 0.1524) (layer F.Cu) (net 18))
 (via (at 92.55 81.45) (size 0.5) (drill 0.3) (layers F.Cu B.Cu) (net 18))
 (segment (start 100.545 84.1625) (end 100.545 83.175) (width 0.1524) (layer F.Cu) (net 18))
 (segment (start 92.55 81.549004) (end 92.55 81.45) (width 0.1524) (layer B.Cu) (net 18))
 (segment (start 93.553407 82.552411) (end 92.55 81.549004) (width 0.1524) (layer B.Cu) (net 18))
 (segment (start 94.3 87.475) (end 93.00121 87.475) (width 0.1524) (layer F.Cu) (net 17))
 (segment (start 94.825 83) (end 94.825 86.95) (width 0.1524) (layer F.Cu) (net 17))
 (segment (start 94.825 86.95) (end 94.3 87.475) (width 0.1524) (layer F.Cu) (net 17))
 (segment (start 96.45 82.725) (end 95.1 82.725) (width 0.1524) (layer F.Cu) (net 17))
 (segment (start 96.735 83.01) (end 96.45 82.725) (width 0.1524) (layer F.Cu) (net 17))
 (segment (start 95.1 82.725) (end 94.825 83) (width 0.1524) (layer F.Cu) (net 17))
 (segment (start 96.735 84.1625) (end 96.735 83.01) (width 0.1524) (layer F.Cu) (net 17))
 (segment (start 95.125 88.125) (end 92.925 88.125) (width 0.1524) (layer F.Cu) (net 11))
 (segment (start 95.465 87.785) (end 95.125 88.125) (width 0.1524) (layer F.Cu) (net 11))
 (segment (start 95.465 84.1625) (end 95.465 87.785) (width 0.1524) (layer F.Cu) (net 11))
 (via (at 91.7 82.5) (size 0.5) (drill 0.3) (layers F.Cu B.Cu) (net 16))
 (segment (start 91.7 84.1175) (end 91.655 84.1625) (width 0.1524) (layer F.Cu) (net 16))
 (segment (start 91.7 82.5) (end 91.7 84.1175) (width 0.1524) (layer F.Cu) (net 16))
 (segment (start 93.3024 88.775) (end 93.6 88.4774) (width 0.1524) (layer B.Cu) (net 16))
 (segment (start 92.925 88.775) (end 93.3024 88.775) (width 0.1524) (layer B.Cu) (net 16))
 (segment (start 93.6 88.4774) (end 93.6 84.4) (width 0.1524) (layer B.Cu) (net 16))
 (segment (start 93.6 84.4) (end 91.7 82.5) (width 0.1524) (layer B.Cu) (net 16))
 (via (at 91.65 78.95) (size 0.5) (drill 0.3) (layers F.Cu B.Cu) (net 15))
 (segment (start 91.65 77.2425) (end 91.655 77.2375) (width 0.1524) (layer F.Cu) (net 15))
 (segment (start 91.65 78.95) (end 91.65 77.2425) (width 0.1524) (layer F.Cu) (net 15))
 (segment (start 93.95241 88.77499) (end 93.95241 83.80241) (width 0.1524) (layer B.Cu) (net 15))
 (segment (start 91.65 81.5) (end 91.65 78.95) (width 0.1524) (layer B.Cu) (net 15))
 (segment (start 93.3024 89.425) (end 93.95241 88.77499) (width 0.1524) (layer B.Cu) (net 15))
 (segment (start 93.95241 83.80241) (end 91.65 81.5) (width 0.1524) (layer B.Cu) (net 15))
 (segment (start 93.3024 89.425) (end 92.7 89.425) (width 0.1524) (layer B.Cu) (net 15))
 (segment (start 93.625 90.075) (end 94 89.7) (width 0.1524) (layer B.Cu) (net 14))
 (segment (start 92.925 90.075) (end 93.625 90.075) (width 0.1524) (layer B.Cu) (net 14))
 (segment (start 95.465 78.585) (end 93.15 80.9) (width 0.1524) (layer F.Cu) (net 14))
 (via (at 93.15 80.9) (size 0.5) (drill 0.3) (layers F.Cu B.Cu) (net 14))
 (segment (start 95.465 77.2375) (end 95.465 78.585) (width 0.1524) (layer F.Cu) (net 14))
 (segment (start 94.30482 89.39518) (end 94.30482 82.05482) (width 0.1524) (layer B.Cu) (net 14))
 (segment (start 94 89.7) (end 94.30482 89.39518) (width 0.1524) (layer B.Cu) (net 14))
 (segment (start 94.30482 82.05482) (end 93.15 80.9) (width 0.1524) (layer B.Cu) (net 14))
 (segment (start 93.753778 90.725) (end 94.178778 90.3) (width 0.1524) (layer B.Cu) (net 13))
 (segment (start 92.925 90.725) (end 93.753778 90.725) (width 0.1524) (layer B.Cu) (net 13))
 (via (at 94.05 80.9) (size 0.5) (drill 0.3) (layers F.Cu B.Cu) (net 13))
 (segment (start 94.85 81.7) (end 94.05 80.9) (width 0.1524) (layer B.Cu) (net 13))
 (segment (start 96.735 78.215) (end 94.05 80.9) (width 0.1524) (layer F.Cu) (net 13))
 (segment (start 96.735 77.2375) (end 96.735 78.215) (width 0.1524) (layer F.Cu) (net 13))
 (segment (start 94.2 90.3) (end 94.85 89.65) (width 0.1524) (layer B.Cu) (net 13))
 (segment (start 94.178778 90.3) (end 94.2 90.3) (width 0.1524) (layer B.Cu) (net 13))
 (segment (start 94.85 89.65) (end 94.85 81.7) (width 0.1524) (layer B.Cu) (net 13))
 (via (at 95.4 80.9) (size 0.5) (drill 0.3) (layers F.Cu B.Cu) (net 12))
 (segment (start 94.675 91.375) (end 92.925 91.375) (width 0.1524) (layer B.Cu) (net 12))
 (segment (start 95.4 90.65) (end 94.675 91.375) (width 0.1524) (layer B.Cu) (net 12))
 (segment (start 95.4 80.9) (end 95.4 90.65) (width 0.1524) (layer B.Cu) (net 12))
 (segment (start 100.545 78.433778) (end 100.545 77.2375) (width 0.1524) (layer F.Cu) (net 12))
 (segment (start 98.978778 80) (end 100.545 78.433778) (width 0.1524) (layer F.Cu) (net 12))
 (segment (start 96.3 80) (end 98.978778 80) (width 0.1524) (layer F.Cu) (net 12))
 (segment (start 95.4 80.9) (end 96.3 80) (width 0.1524) (layer F.Cu) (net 12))
 (segment (start 90.35 84.1275) (end 90.385 84.1625) (width 0.1524) (layer F.Cu) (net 19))
 (segment (start 90.35 82.7) (end 90.35 84.1275) (width 0.1524) (layer F.Cu) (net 19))
 (via (at 90.35 82.5) (size 0.5) (drill 0.3) (layers F.Cu B.Cu) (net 19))
 (segment (start 90.35 82.7) (end 90.35 82.5) (width 0.1524) (layer F.Cu) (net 19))
 (segment (start 90.7 82.5) (end 90.35 82.5) (width 0.1524) (layer B.Cu) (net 19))
 (segment (start 93.2 85) (end 90.7 82.5) (width 0.1524) (layer B.Cu) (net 19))
 (segment (start 93.2 85.9) (end 93.2 85) (width 0.1524) (layer B.Cu) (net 19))
 (segment (start 92.925 86.175) (end 93.2 85.9) (width 0.1524) (layer B.Cu) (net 19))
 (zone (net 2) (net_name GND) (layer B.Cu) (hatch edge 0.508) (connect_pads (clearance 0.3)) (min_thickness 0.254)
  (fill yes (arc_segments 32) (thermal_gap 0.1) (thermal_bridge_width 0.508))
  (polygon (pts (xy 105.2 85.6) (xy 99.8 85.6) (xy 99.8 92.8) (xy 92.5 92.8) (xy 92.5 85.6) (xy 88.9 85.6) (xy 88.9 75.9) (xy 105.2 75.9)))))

